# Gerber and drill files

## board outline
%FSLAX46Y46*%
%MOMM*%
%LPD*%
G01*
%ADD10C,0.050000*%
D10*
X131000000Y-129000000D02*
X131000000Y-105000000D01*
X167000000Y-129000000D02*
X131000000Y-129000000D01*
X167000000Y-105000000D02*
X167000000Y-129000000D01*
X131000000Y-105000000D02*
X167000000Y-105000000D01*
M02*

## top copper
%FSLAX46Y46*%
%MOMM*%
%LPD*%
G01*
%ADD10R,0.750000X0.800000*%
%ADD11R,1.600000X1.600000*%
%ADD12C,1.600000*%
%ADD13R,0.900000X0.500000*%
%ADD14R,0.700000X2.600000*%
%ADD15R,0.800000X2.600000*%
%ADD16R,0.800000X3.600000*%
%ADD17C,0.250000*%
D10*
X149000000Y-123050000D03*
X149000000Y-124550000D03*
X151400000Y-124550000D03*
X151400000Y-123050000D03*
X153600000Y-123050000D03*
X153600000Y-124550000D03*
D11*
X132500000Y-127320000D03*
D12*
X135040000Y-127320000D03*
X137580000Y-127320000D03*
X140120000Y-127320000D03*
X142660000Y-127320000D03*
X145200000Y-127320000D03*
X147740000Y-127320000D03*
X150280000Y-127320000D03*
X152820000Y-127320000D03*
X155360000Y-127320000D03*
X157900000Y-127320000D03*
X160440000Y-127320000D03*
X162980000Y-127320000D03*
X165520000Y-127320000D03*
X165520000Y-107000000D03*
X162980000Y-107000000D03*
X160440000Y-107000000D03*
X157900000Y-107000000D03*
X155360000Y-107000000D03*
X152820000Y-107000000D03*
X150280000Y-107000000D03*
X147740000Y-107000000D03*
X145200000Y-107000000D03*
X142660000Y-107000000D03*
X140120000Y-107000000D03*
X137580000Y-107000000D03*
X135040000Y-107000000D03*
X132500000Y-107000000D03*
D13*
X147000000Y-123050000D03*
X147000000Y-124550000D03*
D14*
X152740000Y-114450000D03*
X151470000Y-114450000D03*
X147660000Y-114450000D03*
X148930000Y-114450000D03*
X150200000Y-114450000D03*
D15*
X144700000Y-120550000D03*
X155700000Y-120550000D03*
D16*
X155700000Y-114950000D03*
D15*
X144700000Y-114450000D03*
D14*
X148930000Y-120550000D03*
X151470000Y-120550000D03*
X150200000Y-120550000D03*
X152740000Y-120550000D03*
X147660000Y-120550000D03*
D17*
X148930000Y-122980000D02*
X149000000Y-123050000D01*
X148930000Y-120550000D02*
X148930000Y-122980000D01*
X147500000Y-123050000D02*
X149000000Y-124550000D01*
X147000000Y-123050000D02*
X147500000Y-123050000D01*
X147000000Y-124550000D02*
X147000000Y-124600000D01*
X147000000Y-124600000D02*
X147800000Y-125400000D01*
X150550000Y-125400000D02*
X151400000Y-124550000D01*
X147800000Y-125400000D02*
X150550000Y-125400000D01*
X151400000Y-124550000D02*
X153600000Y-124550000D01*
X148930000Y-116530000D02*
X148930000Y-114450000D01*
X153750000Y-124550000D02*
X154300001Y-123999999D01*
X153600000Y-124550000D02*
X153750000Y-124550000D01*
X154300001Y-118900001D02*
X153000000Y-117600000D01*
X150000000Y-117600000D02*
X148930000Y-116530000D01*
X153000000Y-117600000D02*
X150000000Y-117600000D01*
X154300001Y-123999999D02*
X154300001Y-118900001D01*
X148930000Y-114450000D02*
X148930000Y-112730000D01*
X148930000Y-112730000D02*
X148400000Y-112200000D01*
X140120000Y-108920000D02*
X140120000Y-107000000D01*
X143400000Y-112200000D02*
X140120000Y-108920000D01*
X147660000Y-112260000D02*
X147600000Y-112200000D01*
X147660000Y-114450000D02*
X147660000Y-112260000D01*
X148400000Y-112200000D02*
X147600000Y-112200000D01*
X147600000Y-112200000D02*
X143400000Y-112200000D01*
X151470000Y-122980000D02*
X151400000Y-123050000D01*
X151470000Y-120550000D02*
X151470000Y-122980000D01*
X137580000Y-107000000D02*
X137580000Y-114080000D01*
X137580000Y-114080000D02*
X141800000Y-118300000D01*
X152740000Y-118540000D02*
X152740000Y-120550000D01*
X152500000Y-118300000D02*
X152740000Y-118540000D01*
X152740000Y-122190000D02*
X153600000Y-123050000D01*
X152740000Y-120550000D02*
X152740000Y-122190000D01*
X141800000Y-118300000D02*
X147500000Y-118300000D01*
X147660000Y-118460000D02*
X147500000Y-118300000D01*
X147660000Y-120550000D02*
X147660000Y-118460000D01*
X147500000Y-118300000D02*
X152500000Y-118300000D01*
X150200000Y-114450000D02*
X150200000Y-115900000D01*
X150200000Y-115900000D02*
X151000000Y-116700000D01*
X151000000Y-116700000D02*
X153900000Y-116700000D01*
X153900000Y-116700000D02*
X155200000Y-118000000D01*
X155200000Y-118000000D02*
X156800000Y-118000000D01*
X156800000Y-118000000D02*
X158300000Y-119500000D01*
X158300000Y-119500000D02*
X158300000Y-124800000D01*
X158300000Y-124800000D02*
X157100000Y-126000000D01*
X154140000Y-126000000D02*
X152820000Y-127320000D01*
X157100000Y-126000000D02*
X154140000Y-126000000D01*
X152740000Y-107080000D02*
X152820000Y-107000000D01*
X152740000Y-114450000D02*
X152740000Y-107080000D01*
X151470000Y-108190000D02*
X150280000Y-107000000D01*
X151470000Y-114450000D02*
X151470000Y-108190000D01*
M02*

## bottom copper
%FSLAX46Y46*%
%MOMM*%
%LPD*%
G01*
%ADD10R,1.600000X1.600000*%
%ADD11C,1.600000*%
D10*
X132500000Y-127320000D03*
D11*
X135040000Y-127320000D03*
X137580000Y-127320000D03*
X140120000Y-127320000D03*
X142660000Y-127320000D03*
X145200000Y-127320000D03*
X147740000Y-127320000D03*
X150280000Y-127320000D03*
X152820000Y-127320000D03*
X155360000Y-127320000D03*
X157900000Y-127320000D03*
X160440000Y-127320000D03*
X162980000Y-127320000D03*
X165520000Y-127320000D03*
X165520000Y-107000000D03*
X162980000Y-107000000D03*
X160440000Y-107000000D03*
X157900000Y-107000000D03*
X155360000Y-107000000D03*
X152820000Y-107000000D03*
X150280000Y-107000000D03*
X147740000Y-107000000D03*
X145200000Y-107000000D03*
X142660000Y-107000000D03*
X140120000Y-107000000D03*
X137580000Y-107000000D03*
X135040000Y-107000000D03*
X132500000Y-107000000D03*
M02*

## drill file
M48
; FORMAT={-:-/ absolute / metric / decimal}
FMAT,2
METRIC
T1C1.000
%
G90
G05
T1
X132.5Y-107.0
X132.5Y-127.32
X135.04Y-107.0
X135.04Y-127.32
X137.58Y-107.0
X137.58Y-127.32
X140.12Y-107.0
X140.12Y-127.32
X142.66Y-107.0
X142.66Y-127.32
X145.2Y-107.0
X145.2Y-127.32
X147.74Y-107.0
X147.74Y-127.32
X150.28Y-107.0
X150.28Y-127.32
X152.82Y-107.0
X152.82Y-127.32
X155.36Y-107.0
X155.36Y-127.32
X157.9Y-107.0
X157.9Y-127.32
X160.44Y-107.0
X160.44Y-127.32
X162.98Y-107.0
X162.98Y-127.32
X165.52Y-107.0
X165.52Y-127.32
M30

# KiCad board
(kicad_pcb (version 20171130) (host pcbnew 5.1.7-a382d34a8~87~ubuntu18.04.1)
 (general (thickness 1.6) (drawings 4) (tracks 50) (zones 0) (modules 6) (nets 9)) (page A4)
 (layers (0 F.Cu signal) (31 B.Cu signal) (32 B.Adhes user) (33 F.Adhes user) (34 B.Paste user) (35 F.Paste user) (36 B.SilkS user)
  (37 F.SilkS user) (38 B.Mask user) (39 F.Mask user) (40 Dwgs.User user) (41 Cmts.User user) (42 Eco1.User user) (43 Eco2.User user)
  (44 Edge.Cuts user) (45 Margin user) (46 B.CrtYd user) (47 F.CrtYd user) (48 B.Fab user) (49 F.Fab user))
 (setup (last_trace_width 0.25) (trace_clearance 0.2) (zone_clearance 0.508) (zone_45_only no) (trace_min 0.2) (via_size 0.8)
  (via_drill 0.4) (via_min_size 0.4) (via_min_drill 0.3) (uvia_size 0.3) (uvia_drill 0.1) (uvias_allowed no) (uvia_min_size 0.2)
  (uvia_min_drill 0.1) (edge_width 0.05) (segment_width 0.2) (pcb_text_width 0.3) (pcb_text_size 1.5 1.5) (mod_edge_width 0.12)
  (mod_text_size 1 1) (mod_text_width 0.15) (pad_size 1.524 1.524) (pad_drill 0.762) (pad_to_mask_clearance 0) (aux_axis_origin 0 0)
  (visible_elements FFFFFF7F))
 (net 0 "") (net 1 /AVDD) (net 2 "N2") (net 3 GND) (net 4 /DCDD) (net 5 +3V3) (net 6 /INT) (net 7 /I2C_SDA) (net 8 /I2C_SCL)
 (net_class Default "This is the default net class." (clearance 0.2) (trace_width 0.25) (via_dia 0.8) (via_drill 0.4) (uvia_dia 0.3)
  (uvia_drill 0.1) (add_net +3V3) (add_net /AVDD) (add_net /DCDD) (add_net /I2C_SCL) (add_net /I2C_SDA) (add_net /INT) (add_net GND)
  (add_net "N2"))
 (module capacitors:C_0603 (layer F.Cu) (at 149 123.8 270)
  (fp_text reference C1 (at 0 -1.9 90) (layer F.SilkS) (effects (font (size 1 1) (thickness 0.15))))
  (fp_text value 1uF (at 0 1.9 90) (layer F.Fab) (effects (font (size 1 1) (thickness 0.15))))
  (pad 1 smd rect (at -0.75 0 270) (size 0.8 0.75) (layers F.Cu F.Paste F.Mask) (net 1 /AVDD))
  (pad 2 smd rect (at 0.75 0 270) (size 0.8 0.75) (layers F.Cu F.Paste F.Mask) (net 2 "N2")))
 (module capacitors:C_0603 (layer F.Cu) (at 151.4 123.8 270)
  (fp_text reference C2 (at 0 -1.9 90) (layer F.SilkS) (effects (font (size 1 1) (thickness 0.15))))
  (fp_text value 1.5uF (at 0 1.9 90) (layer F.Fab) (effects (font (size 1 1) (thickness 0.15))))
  (pad 2 smd rect (at 0.75 0 270) (size 0.8 0.75) (layers F.Cu F.Paste F.Mask) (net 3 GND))
  (pad 1 smd rect (at -0.75 0 270) (size 0.8 0.75) (layers F.Cu F.Paste F.Mask) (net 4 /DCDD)))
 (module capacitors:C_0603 (layer F.Cu) (at 153.6 123.8 270)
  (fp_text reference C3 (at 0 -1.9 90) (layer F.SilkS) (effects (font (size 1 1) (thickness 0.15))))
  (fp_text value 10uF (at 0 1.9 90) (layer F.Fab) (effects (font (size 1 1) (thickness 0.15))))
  (pad 1 smd rect (at -0.75 0 270) (size 0.8 0.75) (layers F.Cu F.Paste F.Mask) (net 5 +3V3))
  (pad 2 smd rect (at 0.75 0 270) (size 0.8 0.75) (layers F.Cu F.Paste F.Mask) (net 3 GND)))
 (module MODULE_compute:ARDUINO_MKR (layer F.Cu) (at 149.01 117.16)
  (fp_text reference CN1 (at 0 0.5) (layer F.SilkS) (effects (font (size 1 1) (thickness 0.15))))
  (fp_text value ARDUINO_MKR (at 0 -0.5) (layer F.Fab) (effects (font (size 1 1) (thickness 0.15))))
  (pad 1 thru_hole rect (at -16.51 10.16) (size 1.6 1.6) (drill 1) (layers *.Cu *.Mask F.SilkS))
  (pad 2 thru_hole circle (at -13.97 10.16) (size 1.6 1.6) (drill 1) (layers *.Cu *.Mask F.SilkS))
  (pad 3 thru_hole circle (at -11.43 10.16) (size 1.6 1.6) (drill 1) (layers *.Cu *.Mask F.SilkS))
  (pad 4 thru_hole circle (at -8.89 10.16) (size 1.6 1.6) (drill 1) (layers *.Cu *.Mask F.SilkS))
  (pad 5 thru_hole circle (at -6.35 10.16) (size 1.6 1.6) (drill 1) (layers *.Cu *.Mask F.SilkS))
  (pad 6 thru_hole circle (at -3.81 10.16) (size 1.6 1.6) (drill 1) (layers *.Cu *.Mask F.SilkS))
  (pad 7 thru_hole circle (at -1.27 10.16) (size 1.6 1.6) (drill 1) (layers *.Cu *.Mask F.SilkS))
  (pad 8 thru_hole circle (at 1.27 10.16) (size 1.6 1.6) (drill 1) (layers *.Cu *.Mask F.SilkS))
  (pad 9 thru_hole circle (at 3.81 10.16) (size 1.6 1.6) (drill 1) (layers *.Cu *.Mask F.SilkS) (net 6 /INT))
  (pad 10 thru_hole circle (at 6.35 10.16) (size 1.6 1.6) (drill 1) (layers *.Cu *.Mask F.SilkS))
  (pad 11 thru_hole circle (at 8.89 10.16) (size 1.6 1.6) (drill 1) (layers *.Cu *.Mask F.SilkS))
  (pad 12 thru_hole circle (at 11.43 10.16) (size 1.6 1.6) (drill 1) (layers *.Cu *.Mask F.SilkS))
  (pad 13 thru_hole circle (at 13.97 10.16) (size 1.6 1.6) (drill 1) (layers *.Cu *.Mask F.SilkS))
  (pad 14 thru_hole circle (at 16.51 10.16) (size 1.6 1.6) (drill 1) (layers *.Cu *.Mask F.SilkS))
  (pad 15 thru_hole circle (at 16.51 -10.16) (size 1.6 1.6) (drill 1) (layers *.Cu *.Mask F.SilkS))
  (pad 16 thru_hole circle (at 13.97 -10.16) (size 1.6 1.6) (drill 1) (layers *.Cu *.Mask F.SilkS))
  (pad 17 thru_hole circle (at 11.43 -10.16) (size 1.6 1.6) (drill 1) (layers *.Cu *.Mask F.SilkS))
  (pad 18 thru_hole circle (at 8.89 -10.16) (size 1.6 1.6) (drill 1) (layers *.Cu *.Mask F.SilkS))
  (pad 19 thru_hole circle (at 6.35 -10.16) (size 1.6 1.6) (drill 1) (layers *.Cu *.Mask F.SilkS))
  (pad 20 thru_hole circle (at 3.81 -10.16) (size 1.6 1.6) (drill 1) (layers *.Cu *.Mask F.SilkS) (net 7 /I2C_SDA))
  (pad 21 thru_hole circle (at 1.27 -10.16) (size 1.6 1.6) (drill 1) (layers *.Cu *.Mask F.SilkS) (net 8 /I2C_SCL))
  (pad 22 thru_hole circle (at -1.27 -10.16) (size 1.6 1.6) (drill 1) (layers *.Cu *.Mask F.SilkS))
  (pad 23 thru_hole circle (at -3.81 -10.16) (size 1.6 1.6) (drill 1) (layers *.Cu *.Mask F.SilkS))
  (pad 24 thru_hole circle (at -6.35 -10.16) (size 1.6 1.6) (drill 1) (layers *.Cu *.Mask F.SilkS))
  (pad 25 thru_hole circle (at -8.89 -10.16) (size 1.6 1.6) (drill 1) (layers *.Cu *.Mask F.SilkS) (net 3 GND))
  (pad 26 thru_hole circle (at -11.43 -10.16) (size 1.6 1.6) (drill 1) (layers *.Cu *.Mask F.SilkS) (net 5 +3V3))
  (pad 27 thru_hole circle (at -13.97 -10.16) (size 1.6 1.6) (drill 1) (layers *.Cu *.Mask F.SilkS))
  (pad 28 thru_hole circle (at -16.51 -10.16) (size 1.6 1.6) (drill 1) (layers *.Cu *.Mask F.SilkS)))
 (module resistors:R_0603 (layer F.Cu) (at 147 123.8 270)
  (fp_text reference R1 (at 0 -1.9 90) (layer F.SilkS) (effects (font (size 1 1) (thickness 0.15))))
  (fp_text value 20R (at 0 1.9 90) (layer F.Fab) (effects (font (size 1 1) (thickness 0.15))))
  (pad 1 smd rect (at -0.75 0 270) (size 0.5 0.9) (layers F.Cu F.Paste F.Mask) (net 2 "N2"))
  (pad 2 smd rect (at 0.75 0 270) (size 0.5 0.9) (layers F.Cu F.Paste F.Mask) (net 3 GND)))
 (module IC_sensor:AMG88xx (layer F.Cu) (at 150.2 117.5 180)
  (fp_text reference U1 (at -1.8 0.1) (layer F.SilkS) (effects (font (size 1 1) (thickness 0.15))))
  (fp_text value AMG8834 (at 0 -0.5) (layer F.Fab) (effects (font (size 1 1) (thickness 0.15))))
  (pad 2 smd rect (at -2.54 3.05 180) (size 0.7 2.6) (layers F.Cu F.Paste F.Mask) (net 7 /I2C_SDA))
  (pad 3 smd rect (at -1.27 3.05 180) (size 0.7 2.6) (layers F.Cu F.Paste F.Mask) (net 8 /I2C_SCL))
  (pad 6 smd rect (at 2.54 3.05 180) (size 0.7 2.6) (layers F.Cu F.Paste F.Mask) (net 3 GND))
  (pad 5 smd rect (at 1.27 3.05 180) (size 0.7 2.6) (layers F.Cu F.Paste F.Mask) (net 3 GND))
  (pad 4 smd rect (at 0 3.05 180) (size 0.7 2.6) (layers F.Cu F.Paste F.Mask) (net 6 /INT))
  (pad 8 smd rect (at 5.5 -3.05 180) (size 0.8 2.6) (layers F.Cu F.Paste F.Mask))
  (pad 14 smd rect (at -5.5 -3.05 180) (size 0.8 2.6) (layers F.Cu F.Paste F.Mask))
  (pad 1 smd rect (at -5.5 2.55 180) (size 0.8 3.6) (layers F.Cu F.Paste F.Mask))
  (pad 7 smd rect (at 5.5 3.05 180) (size 0.8 2.6) (layers F.Cu F.Paste F.Mask))
  (pad 10 smd rect (at 1.27 -3.05 180) (size 0.7 2.6) (layers F.Cu F.Paste F.Mask) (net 1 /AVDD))
  (pad 12 smd rect (at -1.27 -3.05 180) (size 0.7 2.6) (layers F.Cu F.Paste F.Mask) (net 4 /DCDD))
  (pad 11 smd rect (at 0 -3.05 180) (size 0.7 2.6) (layers F.Cu F.Paste F.Mask))
  (pad 13 smd rect (at -2.54 -3.05 180) (size 0.7 2.6) (layers F.Cu F.Paste F.Mask) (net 5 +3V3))
  (pad 9 smd rect (at 2.54 -3.05 180) (size 0.7 2.6) (layers F.Cu F.Paste F.Mask) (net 5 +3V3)))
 (gr_line (start 131 129) (end 131 105) (layer Edge.Cuts) (width 0.05))
 (gr_line (start 167 129) (end 131 129) (layer Edge.Cuts) (width 0.05))
 (gr_line (start 167 105) (end 167 129) (layer Edge.Cuts) (width 0.05))
 (gr_line (start 131 105) (end 167 105) (layer Edge.Cuts) (width 0.05))
 (segment (start 148.93 122.98) (end 149 123.05) (width 0.25) (layer F.Cu) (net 1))
 (segment (start 148.93 120.55) (end 148.93 122.98) (width 0.25) (layer F.Cu) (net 1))
 (segment (start 147.5 123.05) (end 149 124.55) (width 0.25) (layer F.Cu) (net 2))
 (segment (start 147 123.05) (end 147.5 123.05) (width 0.25) (layer F.Cu) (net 2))
 (segment (start 147 124.55) (end 147 124.6) (width 0.25) (layer F.Cu) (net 3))
 (segment (start 147 124.6) (end 147.8 125.4) (width 0.25) (layer F.Cu) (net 3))
 (segment (start 150.55 125.4) (end 151.4 124.55) (width 0.25) (layer F.Cu) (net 3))
 (segment (start 147.8 125.4) (end 150.55 125.4) (width 0.25) (layer F.Cu) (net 3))
 (segment (start 151.4 124.55) (end 153.6 124.55) (width 0.25) (layer F.Cu) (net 3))
 (segment (start 148.93 116.53) (end 148.93 114.45) (width 0.25) (layer F.Cu) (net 3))
 (segment (start 153.75 124.55) (end 154.300001 123.999999) (width 0.25) (layer F.Cu) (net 3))
 (segment (start 153.6 124.55) (end 153.75 124.55) (width 0.25) (layer F.Cu) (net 3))
 (segment (start 154.300001 118.900001) (end 153 117.6) (width 0.25) (layer F.Cu) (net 3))
 (segment (start 150 117.6) (end 148.93 116.53) (width 0.25) (layer F.Cu) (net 3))
 (segment (start 153 117.6) (end 150 117.6) (width 0.25) (layer F.Cu) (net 3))
 (segment (start 154.300001 123.999999) (end 154.300001 118.900001) (width 0.25) (layer F.Cu) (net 3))
 (segment (start 148.93 114.45) (end 148.93 112.73) (width 0.25) (layer F.Cu) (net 3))
 (segment (start 148.93 112.73) (end 148.4 112.2) (width 0.25) (layer F.Cu) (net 3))
 (segment (start 140.12 108.92) (end 140.12 107) (width 0.25) (layer F.Cu) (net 3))
 (segment (start 143.4 112.2) (end 140.12 108.92) (width 0.25) (layer F.Cu) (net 3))
 (segment (start 147.66 112.26) (end 147.6 112.2) (width 0.25) (layer F.Cu) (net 3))
 (segment (start 147.66 114.45) (end 147.66 112.26) (width 0.25) (layer F.Cu) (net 3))
 (segment (start 148.4 112.2) (end 147.6 112.2) (width 0.25) (layer F.Cu) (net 3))
 (segment (start 147.6 112.2) (end 143.4 112.2) (width 0.25) (layer F.Cu) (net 3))
 (segment (start 151.47 122.98) (end 151.4 123.05) (width 0.25) (layer F.Cu) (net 4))
 (segment (start 151.47 120.55) (end 151.47 122.98) (width 0.25) (layer F.Cu) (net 4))
 (segment (start 137.58 107) (end 137.58 114.08) (width 0.25) (layer F.Cu) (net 5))
 (segment (start 137.58 114.08) (end 141.8 118.3) (width 0.25) (layer F.Cu) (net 5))
 (segment (start 152.74 118.54) (end 152.74 120.55) (width 0.25) (layer F.Cu) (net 5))
 (segment (start 152.5 118.3) (end 152.74 118.54) (width 0.25) (layer F.Cu) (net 5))
 (segment (start 152.74 122.19) (end 153.6 123.05) (width 0.25) (layer F.Cu) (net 5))
 (segment (start 152.74 120.55) (end 152.74 122.19) (width 0.25) (layer F.Cu) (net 5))
 (segment (start 141.8 118.3) (end 147.5 118.3) (width 0.25) (layer F.Cu) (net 5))
 (segment (start 147.66 118.46) (end 147.5 118.3) (width 0.25) (layer F.Cu) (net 5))
 (segment (start 147.66 120.55) (end 147.66 118.46) (width 0.25) (layer F.Cu) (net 5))
 (segment (start 147.5 118.3) (end 152.5 118.3) (width 0.25) (layer F.Cu) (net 5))
 (segment (start 150.2 114.45) (end 150.2 115.9) (width 0.25) (layer F.Cu) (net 6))
 (segment (start 150.2 115.9) (end 151 116.7) (width 0.25) (layer F.Cu) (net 6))
 (segment (start 151 116.7) (end 153.9 116.7) (width 0.25) (layer F.Cu) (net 6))
 (segment (start 153.9 116.7) (end 155.2 118) (width 0.25) (layer F.Cu) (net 6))
 (segment (start 155.2 118) (end 156.8 118) (width 0.25) (layer F.Cu) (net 6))
 (segment (start 156.8 118) (end 158.3 119.5) (width 0.25) (layer F.Cu) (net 6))
 (segment (start 158.3 119.5) (end 158.3 124.8) (width 0.25) (layer F.Cu) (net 6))
 (segment (start 158.3 124.8) (end 157.1 126) (width 0.25) (layer F.Cu) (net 6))
 (segment (start 154.14 126) (end 152.82 127.32) (width 0.25) (layer F.Cu) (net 6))
 (segment (start 157.1 126) (end 154.14 126) (width 0.25) (layer F.Cu) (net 6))
 (segment (start 152.74 107.08) (end 152.82 107) (width 0.25) (layer F.Cu) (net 7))
 (segment (start 152.74 114.45) (end 152.74 107.08) (width 0.25) (layer F.Cu) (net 7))
 (segment (start 151.47 108.19) (end 150.28 107) (width 0.25) (layer F.Cu) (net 8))
 (segment (start 151.47 114.45) (end 151.47 108.19) (width 0.25) (layer F.Cu) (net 8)))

